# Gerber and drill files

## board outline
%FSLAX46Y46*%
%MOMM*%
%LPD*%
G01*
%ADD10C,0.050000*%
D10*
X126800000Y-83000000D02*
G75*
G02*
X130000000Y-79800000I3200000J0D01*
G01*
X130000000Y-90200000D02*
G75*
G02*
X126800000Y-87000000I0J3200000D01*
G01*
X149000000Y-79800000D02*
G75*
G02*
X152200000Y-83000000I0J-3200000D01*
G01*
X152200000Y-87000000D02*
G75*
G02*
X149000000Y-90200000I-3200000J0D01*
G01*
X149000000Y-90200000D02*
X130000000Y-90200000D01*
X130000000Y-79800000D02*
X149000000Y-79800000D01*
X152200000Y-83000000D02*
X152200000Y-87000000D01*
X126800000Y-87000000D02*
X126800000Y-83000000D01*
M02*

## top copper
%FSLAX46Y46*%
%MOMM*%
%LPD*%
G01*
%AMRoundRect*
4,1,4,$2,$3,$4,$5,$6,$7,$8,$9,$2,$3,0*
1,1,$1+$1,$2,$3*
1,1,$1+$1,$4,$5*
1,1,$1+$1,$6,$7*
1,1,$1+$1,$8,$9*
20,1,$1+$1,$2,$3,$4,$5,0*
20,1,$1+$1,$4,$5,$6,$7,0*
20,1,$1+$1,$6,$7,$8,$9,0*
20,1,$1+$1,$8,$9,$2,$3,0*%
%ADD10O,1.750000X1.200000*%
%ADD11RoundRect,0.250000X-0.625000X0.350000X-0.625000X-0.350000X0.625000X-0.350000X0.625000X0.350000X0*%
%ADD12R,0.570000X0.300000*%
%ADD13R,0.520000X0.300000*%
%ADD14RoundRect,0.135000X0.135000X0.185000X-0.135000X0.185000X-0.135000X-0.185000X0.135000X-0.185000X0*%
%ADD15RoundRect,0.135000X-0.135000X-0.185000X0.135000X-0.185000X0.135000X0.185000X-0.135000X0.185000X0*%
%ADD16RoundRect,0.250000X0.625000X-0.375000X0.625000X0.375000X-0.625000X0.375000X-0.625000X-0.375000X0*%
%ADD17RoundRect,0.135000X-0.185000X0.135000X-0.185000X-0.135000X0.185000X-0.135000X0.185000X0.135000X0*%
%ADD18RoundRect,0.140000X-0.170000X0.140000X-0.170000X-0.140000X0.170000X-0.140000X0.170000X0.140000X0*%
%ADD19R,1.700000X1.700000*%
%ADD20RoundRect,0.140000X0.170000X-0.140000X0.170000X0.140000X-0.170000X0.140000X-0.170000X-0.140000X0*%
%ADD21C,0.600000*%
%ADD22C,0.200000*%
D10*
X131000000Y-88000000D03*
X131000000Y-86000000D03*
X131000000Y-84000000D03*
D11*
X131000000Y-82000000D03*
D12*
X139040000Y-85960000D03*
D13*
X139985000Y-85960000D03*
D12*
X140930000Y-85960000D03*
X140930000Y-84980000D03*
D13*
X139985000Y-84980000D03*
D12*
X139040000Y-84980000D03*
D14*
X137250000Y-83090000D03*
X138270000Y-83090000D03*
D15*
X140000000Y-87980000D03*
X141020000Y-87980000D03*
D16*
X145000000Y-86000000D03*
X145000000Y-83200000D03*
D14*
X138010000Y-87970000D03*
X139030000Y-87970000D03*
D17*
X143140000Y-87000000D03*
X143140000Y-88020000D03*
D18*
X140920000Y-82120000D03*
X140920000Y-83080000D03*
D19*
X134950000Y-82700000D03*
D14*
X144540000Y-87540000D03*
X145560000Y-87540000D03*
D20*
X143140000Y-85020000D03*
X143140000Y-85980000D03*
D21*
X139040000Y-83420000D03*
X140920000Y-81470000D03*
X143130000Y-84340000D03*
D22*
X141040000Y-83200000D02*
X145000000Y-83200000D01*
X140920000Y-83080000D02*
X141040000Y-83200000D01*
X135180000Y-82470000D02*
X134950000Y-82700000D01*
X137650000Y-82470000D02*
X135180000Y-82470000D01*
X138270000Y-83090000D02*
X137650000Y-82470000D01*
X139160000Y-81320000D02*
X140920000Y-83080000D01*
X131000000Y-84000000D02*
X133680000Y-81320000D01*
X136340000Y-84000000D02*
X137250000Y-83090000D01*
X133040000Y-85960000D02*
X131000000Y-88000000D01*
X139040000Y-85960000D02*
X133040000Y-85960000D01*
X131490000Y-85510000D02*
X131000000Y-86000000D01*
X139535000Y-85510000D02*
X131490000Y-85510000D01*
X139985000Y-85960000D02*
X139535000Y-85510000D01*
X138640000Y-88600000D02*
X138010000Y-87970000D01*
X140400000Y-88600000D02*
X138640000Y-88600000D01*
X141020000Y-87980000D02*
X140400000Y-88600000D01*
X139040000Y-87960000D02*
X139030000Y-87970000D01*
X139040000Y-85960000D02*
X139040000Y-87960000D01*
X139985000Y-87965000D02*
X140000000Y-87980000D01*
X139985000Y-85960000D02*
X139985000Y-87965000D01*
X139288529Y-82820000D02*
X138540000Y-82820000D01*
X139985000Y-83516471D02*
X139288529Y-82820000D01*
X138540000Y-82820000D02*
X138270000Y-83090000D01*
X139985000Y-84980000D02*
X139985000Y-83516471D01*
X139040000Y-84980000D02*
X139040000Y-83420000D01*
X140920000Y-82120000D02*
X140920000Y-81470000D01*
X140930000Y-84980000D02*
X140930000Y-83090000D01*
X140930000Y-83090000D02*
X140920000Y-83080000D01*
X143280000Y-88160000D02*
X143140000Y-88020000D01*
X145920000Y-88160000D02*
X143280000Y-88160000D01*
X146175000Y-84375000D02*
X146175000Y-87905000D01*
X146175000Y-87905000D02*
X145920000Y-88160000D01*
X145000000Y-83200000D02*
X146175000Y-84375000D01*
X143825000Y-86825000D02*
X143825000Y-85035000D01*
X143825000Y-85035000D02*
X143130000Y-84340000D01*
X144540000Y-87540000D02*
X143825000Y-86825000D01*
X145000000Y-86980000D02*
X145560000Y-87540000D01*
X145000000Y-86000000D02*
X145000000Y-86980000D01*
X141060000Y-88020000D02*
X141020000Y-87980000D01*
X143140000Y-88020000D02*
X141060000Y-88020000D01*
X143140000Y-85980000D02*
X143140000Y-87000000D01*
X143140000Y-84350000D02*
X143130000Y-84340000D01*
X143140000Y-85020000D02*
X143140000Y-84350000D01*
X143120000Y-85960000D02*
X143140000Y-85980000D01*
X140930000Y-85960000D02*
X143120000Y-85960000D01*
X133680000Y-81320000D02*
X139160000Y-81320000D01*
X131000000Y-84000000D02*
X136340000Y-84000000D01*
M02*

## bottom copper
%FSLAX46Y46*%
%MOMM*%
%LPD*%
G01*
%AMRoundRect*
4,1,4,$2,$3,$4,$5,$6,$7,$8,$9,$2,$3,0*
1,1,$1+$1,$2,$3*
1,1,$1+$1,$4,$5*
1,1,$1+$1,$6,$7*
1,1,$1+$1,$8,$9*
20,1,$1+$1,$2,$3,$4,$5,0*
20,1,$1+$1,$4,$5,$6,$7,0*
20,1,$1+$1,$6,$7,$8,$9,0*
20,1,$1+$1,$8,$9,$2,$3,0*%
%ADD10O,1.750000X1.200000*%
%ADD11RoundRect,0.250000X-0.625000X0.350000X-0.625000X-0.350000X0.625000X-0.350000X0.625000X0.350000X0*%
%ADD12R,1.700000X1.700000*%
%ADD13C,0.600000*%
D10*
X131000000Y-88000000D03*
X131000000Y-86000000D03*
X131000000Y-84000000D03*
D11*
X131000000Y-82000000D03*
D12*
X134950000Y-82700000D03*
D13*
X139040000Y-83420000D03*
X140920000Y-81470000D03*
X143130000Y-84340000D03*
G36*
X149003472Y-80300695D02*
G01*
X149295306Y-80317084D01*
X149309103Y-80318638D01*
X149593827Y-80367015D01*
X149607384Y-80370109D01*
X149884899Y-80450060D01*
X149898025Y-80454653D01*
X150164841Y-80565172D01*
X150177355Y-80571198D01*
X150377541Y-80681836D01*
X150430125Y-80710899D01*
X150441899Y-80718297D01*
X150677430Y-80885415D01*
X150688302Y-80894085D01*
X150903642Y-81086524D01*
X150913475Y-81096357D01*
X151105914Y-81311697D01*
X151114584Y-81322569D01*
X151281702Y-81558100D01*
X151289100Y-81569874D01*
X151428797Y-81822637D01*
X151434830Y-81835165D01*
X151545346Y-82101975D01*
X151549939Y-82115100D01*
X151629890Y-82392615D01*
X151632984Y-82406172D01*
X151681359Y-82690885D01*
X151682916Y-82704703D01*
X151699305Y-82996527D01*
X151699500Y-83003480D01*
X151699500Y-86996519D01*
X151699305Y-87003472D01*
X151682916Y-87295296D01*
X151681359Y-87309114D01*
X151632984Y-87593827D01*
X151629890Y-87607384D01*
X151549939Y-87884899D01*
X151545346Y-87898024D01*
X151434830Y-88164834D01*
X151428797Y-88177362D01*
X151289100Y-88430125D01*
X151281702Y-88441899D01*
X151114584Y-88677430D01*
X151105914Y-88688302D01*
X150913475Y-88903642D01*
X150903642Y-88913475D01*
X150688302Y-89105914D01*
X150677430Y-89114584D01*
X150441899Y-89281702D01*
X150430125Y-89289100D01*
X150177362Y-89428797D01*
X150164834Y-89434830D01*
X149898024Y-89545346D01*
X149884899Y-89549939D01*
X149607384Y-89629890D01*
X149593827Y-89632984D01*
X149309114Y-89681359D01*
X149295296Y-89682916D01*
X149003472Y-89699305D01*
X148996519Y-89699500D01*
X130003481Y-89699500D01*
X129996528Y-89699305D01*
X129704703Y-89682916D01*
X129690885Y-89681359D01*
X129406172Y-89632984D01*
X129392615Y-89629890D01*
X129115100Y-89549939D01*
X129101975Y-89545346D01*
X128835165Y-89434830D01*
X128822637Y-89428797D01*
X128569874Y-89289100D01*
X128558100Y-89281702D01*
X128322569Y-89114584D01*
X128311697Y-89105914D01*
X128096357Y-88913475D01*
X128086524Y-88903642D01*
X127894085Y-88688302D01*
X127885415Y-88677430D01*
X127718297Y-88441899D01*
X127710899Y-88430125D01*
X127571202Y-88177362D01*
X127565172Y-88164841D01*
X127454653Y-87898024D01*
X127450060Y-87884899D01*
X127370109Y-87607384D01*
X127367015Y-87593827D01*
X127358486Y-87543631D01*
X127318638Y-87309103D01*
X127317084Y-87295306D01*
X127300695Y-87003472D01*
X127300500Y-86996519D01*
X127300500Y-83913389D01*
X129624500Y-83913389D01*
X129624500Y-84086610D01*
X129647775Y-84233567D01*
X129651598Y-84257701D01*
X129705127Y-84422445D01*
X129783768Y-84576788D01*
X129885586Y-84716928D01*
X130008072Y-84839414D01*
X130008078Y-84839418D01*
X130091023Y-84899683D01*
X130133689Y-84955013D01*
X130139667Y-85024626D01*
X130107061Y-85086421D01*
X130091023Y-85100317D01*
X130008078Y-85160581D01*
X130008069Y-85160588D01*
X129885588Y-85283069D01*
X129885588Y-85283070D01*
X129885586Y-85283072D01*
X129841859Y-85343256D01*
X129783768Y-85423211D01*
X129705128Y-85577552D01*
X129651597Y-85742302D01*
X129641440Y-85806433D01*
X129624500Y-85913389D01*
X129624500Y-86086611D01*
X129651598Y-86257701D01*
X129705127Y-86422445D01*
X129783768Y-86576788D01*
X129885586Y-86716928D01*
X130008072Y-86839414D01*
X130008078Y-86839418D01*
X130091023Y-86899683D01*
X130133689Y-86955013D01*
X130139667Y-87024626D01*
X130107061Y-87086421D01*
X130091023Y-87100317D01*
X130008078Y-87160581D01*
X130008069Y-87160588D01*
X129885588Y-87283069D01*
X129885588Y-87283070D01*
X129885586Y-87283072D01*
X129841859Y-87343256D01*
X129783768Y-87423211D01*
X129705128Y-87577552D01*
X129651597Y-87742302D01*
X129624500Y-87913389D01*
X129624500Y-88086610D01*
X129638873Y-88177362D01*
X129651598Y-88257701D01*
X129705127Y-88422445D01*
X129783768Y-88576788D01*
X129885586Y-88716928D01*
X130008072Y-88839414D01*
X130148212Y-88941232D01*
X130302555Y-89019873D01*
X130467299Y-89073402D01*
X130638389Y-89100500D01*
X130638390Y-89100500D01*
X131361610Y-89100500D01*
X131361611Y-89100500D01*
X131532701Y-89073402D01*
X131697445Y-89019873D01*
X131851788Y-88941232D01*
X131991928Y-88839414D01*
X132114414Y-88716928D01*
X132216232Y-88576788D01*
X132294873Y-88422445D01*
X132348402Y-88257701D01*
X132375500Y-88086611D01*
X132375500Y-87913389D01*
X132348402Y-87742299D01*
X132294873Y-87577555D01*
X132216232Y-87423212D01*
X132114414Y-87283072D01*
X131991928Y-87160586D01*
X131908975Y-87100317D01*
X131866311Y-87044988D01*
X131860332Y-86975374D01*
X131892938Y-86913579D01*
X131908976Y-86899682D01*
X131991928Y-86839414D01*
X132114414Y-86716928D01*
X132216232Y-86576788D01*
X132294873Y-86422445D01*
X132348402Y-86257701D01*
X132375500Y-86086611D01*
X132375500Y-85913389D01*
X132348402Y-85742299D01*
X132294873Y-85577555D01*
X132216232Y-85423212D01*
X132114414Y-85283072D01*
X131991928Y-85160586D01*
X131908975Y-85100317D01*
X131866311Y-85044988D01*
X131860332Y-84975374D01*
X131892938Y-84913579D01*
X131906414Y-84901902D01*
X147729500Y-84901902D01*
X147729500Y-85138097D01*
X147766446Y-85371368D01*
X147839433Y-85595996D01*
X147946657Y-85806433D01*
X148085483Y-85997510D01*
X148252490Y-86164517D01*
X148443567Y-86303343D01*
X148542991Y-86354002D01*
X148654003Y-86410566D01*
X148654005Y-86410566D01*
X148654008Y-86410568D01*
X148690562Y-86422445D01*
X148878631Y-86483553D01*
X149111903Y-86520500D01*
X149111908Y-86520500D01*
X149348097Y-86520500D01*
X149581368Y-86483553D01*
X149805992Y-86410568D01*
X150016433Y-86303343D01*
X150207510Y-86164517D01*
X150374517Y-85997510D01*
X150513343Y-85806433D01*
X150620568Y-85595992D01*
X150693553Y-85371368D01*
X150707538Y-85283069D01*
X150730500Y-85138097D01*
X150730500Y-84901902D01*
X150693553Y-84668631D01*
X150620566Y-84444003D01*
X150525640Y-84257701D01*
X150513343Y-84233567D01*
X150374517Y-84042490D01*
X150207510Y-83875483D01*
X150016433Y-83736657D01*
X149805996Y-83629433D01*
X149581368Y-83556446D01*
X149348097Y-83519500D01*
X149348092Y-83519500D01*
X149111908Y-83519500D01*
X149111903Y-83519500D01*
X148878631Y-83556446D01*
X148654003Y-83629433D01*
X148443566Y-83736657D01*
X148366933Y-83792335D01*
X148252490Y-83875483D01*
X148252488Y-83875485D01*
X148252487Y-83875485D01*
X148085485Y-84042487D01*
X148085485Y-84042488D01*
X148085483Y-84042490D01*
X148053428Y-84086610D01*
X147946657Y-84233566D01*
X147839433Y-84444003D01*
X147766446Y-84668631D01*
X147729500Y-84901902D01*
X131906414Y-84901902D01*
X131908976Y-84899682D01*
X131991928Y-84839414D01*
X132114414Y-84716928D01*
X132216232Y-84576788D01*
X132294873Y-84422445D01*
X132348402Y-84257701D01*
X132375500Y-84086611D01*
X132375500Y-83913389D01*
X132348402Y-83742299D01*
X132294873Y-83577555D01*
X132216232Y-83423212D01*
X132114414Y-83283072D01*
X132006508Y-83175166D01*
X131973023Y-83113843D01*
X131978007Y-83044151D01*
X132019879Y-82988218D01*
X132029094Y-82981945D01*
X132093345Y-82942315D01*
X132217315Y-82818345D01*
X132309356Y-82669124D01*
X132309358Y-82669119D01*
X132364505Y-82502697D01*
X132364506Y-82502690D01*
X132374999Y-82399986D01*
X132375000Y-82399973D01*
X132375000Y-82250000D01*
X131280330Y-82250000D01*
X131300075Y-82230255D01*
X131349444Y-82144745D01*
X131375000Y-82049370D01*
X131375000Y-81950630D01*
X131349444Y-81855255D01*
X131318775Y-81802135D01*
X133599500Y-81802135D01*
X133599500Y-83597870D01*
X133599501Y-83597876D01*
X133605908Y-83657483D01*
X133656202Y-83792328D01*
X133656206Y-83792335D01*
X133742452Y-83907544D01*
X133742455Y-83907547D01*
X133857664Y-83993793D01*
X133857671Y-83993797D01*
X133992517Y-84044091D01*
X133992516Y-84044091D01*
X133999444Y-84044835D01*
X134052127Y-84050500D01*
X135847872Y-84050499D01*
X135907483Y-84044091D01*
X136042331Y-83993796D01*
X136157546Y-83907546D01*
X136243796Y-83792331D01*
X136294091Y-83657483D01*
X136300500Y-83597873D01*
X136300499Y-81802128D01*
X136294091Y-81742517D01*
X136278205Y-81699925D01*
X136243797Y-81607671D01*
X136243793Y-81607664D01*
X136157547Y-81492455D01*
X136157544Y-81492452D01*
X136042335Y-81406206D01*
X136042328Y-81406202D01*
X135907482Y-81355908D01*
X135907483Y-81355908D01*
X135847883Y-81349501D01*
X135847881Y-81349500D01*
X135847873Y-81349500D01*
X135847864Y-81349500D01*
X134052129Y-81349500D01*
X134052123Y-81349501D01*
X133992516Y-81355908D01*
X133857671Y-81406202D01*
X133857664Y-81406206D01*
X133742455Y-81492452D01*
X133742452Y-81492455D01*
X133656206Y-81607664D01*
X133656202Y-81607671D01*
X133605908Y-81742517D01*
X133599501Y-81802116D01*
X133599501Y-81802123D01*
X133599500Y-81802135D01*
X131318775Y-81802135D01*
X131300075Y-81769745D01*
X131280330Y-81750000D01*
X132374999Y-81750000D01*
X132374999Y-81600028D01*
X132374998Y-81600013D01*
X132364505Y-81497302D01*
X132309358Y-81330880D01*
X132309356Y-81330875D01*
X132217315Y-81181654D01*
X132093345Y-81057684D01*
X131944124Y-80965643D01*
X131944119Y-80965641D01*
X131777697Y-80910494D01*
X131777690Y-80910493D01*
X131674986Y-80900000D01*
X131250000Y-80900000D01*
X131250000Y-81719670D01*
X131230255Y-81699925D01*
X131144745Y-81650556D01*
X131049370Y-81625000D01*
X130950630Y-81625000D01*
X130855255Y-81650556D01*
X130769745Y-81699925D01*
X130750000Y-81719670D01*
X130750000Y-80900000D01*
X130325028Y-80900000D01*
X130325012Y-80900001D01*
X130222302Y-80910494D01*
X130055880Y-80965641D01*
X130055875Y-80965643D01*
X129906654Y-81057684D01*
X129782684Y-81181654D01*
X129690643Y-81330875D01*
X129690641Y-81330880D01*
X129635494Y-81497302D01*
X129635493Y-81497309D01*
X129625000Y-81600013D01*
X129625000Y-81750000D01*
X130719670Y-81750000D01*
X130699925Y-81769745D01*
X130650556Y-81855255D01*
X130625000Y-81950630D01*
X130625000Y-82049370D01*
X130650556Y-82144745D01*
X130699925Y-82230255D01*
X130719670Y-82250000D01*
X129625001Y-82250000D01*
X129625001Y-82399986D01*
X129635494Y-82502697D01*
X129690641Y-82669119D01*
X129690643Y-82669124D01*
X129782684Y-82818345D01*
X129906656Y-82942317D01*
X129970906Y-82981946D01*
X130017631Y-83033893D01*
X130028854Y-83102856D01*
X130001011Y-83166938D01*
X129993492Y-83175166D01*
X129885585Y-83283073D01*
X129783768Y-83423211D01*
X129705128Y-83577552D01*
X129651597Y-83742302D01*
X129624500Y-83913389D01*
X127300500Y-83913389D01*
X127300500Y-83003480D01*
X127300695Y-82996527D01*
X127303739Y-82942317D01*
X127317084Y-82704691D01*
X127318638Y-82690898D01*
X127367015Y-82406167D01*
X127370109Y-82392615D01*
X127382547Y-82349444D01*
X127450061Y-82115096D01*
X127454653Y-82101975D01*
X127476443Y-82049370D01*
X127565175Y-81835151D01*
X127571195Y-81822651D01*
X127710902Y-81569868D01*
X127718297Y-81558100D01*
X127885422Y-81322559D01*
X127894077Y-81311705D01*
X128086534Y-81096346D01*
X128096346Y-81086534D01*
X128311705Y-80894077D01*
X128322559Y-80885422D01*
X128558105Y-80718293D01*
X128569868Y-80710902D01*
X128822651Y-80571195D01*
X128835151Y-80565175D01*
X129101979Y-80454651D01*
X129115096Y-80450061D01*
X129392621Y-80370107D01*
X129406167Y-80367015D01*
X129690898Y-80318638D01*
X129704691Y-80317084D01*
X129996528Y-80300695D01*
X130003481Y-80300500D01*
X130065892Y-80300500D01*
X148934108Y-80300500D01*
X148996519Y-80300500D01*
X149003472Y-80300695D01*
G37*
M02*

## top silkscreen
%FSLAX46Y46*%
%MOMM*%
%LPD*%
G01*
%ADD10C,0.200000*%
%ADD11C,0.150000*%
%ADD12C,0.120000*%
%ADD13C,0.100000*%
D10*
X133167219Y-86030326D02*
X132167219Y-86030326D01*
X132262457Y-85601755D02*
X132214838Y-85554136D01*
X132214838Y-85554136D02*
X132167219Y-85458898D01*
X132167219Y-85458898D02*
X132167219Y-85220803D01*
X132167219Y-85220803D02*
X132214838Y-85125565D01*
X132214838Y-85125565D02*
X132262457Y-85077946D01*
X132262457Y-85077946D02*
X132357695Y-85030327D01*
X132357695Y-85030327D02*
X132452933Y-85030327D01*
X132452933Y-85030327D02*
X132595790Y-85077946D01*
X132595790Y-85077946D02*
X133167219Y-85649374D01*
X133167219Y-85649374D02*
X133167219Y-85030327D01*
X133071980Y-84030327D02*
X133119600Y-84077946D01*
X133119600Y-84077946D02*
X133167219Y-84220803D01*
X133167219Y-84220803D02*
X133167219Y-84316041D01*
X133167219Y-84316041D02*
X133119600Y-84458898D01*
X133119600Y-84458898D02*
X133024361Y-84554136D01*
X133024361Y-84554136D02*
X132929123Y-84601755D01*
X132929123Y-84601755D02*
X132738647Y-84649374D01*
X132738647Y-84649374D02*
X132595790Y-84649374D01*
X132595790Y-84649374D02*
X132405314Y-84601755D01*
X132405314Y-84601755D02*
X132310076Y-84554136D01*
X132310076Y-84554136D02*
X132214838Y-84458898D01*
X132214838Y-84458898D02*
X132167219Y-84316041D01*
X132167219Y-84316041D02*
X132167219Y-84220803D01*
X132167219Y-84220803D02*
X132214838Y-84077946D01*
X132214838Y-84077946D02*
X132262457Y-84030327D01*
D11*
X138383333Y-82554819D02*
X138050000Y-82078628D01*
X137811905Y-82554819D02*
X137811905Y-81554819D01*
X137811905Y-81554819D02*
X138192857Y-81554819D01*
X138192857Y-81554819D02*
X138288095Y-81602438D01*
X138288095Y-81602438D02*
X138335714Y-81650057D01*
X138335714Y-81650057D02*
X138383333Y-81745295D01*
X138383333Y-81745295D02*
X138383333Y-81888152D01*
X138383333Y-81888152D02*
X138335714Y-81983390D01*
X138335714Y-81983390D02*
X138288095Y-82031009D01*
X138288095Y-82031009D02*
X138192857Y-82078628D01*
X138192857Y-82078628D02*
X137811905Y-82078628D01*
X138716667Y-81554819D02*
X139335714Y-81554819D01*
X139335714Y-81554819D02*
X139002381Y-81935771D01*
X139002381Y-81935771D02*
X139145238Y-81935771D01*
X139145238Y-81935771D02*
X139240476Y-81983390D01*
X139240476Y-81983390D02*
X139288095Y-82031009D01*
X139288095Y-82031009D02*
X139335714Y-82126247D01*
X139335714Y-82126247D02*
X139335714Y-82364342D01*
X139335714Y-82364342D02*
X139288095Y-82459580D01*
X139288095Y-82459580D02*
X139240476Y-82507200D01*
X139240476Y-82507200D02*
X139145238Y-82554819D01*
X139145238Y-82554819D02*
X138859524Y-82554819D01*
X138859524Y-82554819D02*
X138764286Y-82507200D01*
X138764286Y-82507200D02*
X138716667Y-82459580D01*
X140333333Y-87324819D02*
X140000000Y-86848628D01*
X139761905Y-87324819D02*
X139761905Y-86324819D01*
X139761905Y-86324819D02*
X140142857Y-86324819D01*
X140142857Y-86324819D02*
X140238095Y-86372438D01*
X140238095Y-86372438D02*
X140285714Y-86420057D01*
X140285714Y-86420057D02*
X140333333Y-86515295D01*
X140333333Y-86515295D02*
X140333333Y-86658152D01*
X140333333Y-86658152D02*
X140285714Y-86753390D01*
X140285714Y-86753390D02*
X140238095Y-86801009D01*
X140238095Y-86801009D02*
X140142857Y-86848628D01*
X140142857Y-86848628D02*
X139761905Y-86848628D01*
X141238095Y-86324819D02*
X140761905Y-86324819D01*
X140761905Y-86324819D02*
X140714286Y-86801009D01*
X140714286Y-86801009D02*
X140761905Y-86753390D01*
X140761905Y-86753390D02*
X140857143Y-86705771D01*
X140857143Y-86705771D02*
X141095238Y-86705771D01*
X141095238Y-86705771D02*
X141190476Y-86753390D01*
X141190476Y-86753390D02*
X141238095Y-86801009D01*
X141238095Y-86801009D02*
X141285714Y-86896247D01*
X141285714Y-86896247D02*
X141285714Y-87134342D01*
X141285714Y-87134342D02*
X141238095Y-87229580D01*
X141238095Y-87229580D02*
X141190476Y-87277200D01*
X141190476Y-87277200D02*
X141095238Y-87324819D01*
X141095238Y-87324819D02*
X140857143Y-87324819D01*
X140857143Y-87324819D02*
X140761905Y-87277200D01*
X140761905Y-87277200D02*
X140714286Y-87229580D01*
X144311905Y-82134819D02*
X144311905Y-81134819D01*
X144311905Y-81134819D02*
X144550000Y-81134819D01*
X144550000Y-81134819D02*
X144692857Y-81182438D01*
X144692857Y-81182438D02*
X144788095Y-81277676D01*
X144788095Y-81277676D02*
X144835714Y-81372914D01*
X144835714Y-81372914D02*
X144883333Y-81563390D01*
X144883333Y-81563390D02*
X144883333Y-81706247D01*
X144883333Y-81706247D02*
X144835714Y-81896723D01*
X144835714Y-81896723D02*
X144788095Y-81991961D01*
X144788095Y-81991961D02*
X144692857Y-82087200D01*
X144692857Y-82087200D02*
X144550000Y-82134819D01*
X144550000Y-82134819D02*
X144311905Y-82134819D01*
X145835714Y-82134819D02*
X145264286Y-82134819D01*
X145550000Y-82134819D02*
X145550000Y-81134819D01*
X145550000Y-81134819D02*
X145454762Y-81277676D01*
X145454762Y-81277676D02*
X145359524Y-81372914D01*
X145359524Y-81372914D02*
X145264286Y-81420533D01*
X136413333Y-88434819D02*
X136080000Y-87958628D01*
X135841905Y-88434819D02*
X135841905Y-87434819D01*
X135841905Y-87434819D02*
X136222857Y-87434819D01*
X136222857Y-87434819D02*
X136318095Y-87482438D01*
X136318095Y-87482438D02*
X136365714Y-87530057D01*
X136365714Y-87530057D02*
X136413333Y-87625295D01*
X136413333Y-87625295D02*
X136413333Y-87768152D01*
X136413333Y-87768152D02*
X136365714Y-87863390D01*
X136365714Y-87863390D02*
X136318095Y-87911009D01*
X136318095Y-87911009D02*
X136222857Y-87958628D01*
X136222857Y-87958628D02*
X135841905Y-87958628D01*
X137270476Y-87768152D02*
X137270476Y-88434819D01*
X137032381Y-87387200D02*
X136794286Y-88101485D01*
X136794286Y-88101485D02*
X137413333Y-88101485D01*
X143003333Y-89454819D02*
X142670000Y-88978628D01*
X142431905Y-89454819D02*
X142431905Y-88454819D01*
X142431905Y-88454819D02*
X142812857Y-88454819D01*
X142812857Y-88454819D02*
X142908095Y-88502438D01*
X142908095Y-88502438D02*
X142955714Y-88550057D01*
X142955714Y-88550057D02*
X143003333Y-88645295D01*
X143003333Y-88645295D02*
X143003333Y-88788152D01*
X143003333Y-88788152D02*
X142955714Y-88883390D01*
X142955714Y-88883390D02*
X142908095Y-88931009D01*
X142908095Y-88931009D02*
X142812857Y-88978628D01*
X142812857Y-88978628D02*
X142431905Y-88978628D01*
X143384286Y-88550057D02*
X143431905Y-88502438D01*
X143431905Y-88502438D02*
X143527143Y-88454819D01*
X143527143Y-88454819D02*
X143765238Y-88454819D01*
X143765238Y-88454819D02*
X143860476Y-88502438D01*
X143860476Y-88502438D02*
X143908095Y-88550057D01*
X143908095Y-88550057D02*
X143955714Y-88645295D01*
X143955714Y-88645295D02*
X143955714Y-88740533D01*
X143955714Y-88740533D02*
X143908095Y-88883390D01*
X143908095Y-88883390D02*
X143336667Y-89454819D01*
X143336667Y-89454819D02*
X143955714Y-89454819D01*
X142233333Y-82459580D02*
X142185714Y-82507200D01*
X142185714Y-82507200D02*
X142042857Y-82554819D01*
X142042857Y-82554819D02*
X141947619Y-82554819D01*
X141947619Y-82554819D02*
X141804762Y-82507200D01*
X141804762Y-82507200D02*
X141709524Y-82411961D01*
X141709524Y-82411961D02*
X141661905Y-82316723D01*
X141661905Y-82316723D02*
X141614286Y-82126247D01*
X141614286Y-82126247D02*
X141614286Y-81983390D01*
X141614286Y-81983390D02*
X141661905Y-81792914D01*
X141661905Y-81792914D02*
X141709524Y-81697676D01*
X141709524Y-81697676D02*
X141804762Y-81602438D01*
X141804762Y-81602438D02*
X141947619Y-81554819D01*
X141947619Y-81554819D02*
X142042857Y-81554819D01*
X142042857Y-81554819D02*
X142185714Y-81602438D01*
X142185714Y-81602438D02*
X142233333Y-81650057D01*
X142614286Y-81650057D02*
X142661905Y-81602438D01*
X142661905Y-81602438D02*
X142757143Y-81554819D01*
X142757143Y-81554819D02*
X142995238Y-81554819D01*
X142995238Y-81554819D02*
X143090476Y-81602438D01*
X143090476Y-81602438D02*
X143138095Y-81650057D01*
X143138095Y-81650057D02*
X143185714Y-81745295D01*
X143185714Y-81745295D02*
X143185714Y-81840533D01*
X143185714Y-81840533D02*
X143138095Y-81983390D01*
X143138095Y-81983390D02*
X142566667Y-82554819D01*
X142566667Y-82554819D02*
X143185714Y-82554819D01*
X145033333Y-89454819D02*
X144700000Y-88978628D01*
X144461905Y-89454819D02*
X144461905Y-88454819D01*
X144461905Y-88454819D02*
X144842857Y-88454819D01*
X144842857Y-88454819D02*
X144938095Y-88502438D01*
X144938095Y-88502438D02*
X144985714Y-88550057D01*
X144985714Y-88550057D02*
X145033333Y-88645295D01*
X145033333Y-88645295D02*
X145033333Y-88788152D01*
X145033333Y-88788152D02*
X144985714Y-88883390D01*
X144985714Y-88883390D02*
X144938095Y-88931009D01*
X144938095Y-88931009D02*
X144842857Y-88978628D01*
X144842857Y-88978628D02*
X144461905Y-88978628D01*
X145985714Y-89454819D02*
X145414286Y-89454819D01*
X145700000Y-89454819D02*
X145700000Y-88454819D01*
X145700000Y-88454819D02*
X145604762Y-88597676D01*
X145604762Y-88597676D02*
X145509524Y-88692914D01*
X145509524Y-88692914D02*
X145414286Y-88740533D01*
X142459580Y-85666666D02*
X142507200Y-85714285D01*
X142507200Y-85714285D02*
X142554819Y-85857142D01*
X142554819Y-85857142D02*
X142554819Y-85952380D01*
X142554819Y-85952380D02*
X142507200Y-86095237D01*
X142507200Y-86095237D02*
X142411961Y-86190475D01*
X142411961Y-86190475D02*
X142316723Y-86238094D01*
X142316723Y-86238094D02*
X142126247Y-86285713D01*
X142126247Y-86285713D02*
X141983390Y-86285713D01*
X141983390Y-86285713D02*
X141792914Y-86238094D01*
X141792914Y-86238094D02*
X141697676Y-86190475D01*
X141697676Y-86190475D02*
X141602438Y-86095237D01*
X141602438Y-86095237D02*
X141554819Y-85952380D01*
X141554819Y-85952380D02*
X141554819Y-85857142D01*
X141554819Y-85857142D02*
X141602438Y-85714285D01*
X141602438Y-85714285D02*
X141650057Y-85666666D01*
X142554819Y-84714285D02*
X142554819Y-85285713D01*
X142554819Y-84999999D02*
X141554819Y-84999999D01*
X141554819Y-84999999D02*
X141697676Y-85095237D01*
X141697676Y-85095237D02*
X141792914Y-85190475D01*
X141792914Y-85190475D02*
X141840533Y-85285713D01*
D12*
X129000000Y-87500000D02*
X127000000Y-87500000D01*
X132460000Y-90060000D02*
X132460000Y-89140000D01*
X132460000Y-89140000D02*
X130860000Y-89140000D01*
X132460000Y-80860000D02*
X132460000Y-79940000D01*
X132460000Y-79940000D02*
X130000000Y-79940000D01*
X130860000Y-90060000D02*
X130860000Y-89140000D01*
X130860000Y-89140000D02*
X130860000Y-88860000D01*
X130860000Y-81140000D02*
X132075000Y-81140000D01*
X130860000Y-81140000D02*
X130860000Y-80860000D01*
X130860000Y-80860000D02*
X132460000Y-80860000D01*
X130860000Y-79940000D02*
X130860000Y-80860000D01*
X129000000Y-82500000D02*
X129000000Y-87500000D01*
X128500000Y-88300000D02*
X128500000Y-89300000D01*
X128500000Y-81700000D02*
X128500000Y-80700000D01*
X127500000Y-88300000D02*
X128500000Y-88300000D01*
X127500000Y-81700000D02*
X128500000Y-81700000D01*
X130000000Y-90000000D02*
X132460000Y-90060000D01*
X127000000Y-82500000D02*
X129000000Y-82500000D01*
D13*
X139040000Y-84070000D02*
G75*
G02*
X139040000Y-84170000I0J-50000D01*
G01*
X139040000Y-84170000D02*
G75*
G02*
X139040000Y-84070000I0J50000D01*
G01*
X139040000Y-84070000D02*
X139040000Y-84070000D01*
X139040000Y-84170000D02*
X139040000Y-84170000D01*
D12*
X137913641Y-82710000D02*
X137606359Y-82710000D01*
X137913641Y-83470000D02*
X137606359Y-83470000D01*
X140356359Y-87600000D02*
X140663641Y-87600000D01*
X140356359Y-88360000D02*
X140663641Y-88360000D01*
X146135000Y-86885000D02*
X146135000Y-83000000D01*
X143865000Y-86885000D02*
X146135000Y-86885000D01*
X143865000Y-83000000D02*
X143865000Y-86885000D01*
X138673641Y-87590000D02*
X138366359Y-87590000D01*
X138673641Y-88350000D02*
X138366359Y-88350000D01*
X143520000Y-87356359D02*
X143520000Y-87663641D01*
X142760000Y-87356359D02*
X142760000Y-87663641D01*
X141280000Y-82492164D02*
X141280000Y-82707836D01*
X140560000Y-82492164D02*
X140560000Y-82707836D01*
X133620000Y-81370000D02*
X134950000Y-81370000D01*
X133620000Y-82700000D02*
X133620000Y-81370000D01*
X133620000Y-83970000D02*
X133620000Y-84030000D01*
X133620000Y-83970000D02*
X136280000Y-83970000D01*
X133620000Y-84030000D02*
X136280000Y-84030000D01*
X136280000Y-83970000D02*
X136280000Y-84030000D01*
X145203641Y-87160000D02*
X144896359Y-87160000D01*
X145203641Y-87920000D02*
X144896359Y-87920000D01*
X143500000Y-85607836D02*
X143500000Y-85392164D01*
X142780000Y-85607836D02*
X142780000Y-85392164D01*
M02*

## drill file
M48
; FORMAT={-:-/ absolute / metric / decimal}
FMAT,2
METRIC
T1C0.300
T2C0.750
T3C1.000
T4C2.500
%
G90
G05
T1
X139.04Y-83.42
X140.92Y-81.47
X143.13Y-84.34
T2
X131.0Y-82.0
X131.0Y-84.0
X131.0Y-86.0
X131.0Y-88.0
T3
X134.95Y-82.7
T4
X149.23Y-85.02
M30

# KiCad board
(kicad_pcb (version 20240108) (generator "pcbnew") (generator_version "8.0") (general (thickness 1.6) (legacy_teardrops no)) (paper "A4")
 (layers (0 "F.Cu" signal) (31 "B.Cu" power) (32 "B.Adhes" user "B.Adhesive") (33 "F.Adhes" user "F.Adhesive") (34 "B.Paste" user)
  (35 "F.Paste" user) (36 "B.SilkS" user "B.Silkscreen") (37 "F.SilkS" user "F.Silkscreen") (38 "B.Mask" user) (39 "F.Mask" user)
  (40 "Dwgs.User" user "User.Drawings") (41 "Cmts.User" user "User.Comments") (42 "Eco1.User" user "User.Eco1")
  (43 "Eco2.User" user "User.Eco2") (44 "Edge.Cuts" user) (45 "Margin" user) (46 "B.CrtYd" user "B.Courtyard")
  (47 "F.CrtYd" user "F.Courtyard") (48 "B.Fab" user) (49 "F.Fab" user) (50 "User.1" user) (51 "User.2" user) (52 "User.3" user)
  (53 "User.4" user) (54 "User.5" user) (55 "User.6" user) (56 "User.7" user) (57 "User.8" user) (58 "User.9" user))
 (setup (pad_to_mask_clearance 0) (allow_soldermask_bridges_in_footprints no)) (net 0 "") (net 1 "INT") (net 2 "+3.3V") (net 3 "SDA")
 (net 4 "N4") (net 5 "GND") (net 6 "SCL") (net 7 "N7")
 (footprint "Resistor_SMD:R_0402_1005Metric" (layer "F.Cu") (at 137.76 83.09 180)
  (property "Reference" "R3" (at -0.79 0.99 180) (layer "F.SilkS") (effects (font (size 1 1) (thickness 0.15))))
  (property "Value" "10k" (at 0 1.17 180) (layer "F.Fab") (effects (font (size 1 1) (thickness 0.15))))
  (fp_line (start -0.153641 0.38) (end 0.153641 0.38) (stroke (width 0.12) (type solid)) (layer "F.SilkS"))
  (fp_line (start -0.153641 -0.38) (end 0.153641 -0.38) (stroke (width 0.12) (type solid)) (layer "F.SilkS"))
  (pad "1" smd roundrect (at -0.51 0 180) (size 0.54 0.64) (layers "F.Cu" "F.Paste" "F.Mask") (roundrect_rratio 0.25) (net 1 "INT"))
  (pad "2" smd roundrect (at 0.51 0 180) (size 0.54 0.64) (layers "F.Cu" "F.Paste" "F.Mask") (roundrect_rratio 0.25) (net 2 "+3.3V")))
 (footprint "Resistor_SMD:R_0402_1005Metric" (layer "F.Cu") (at 140.51 87.98)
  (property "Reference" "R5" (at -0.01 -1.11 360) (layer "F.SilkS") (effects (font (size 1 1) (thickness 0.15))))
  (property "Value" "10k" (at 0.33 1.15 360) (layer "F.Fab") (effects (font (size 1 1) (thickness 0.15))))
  (fp_line (start -0.153641 -0.38) (end 0.153641 -0.38) (stroke (width 0.12) (type solid)) (layer "F.SilkS"))
  (fp_line (start -0.153641 0.38) (end 0.153641 0.38) (stroke (width 0.12) (type solid)) (layer "F.SilkS"))
  (pad "1" smd roundrect (at -0.51 0) (size 0.54 0.64) (layers "F.Cu" "F.Paste" "F.Mask") (roundrect_rratio 0.25) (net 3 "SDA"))
  (pad "2" smd roundrect (at 0.51 0) (size 0.54 0.64) (layers "F.Cu" "F.Paste" "F.Mask") (roundrect_rratio 0.25) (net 2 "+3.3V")))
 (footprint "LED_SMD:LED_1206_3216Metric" (layer "F.Cu") (at 145 84.6 90)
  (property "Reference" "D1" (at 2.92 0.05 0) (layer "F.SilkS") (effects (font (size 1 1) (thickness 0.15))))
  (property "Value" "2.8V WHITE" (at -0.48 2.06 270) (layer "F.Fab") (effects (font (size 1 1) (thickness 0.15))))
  (fp_line (start 1.6 -1.135) (end -2.285 -1.135) (stroke (width 0.12) (type solid)) (layer "F.SilkS"))
  (fp_line (start -2.285 -1.135) (end -2.285 1.135) (stroke (width 0.12) (type solid)) (layer "F.SilkS"))
  (fp_line (start -2.285 1.135) (end 1.6 1.135) (stroke (width 0.12) (type solid)) (layer "F.SilkS"))
  (pad "1" smd roundrect (at -1.4 0 90) (size 1.25 1.75) (layers "F.Cu" "F.Paste" "F.Mask") (roundrect_rratio 0.2) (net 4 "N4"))
  (pad "2" smd roundrect (at 1.4 0 90) (size 1.25 1.75) (layers "F.Cu" "F.Paste" "F.Mask") (roundrect_rratio 0.2) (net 2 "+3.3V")))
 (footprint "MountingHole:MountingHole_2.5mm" (layer "F.Cu") (at 149.23 85.02)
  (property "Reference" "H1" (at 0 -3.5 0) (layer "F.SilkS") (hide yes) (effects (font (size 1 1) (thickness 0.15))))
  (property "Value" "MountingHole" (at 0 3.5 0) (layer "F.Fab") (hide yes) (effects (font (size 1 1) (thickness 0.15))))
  (pad "" np_thru_hole circle (at 0 0) (size 2.5 2.5) (drill 2.5) (layers "*.Cu" "*.Mask")))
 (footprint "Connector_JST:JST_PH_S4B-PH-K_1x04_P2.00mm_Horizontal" (layer "F.Cu") (at 131 82 -90)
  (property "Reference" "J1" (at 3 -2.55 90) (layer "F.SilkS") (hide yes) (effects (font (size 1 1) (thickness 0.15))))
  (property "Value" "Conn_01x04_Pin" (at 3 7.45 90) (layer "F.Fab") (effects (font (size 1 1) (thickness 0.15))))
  (fp_line (start 0.5 4) (end 0.5 2) (stroke (width 0.12) (type solid)) (layer "F.SilkS"))
  (fp_line (start -0.3 3.5) (end -0.3 2.5) (stroke (width 0.12) (type solid)) (layer "F.SilkS"))
  (fp_line (start 6.3 3.5) (end 6.3 2.5) (stroke (width 0.12) (type solid)) (layer "F.SilkS"))
  (fp_line (start -0.3 2.5) (end -1.3 2.5) (stroke (width 0.12) (type solid)) (layer "F.SilkS"))
  (fp_line (start 6.3 2.5) (end 7.3 2.5) (stroke (width 0.12) (type solid)) (layer "F.SilkS"))
  (fp_line (start 0.5 2) (end 5.5 2) (stroke (width 0.12) (type solid)) (layer "F.SilkS"))
  (fp_line (start 5.5 2) (end 5.5 4) (stroke (width 0.12) (type solid)) (layer "F.SilkS"))
  (fp_line (start 8 1) (end 8.06 -1.46) (stroke (width 0.12) (type solid)) (layer "F.SilkS"))
  (fp_line (start -2.06 0.14) (end -1.14 0.14) (stroke (width 0.12) (type solid)) (layer "F.SilkS"))
  (fp_line (start -1.14 0.14) (end -1.14 -1.46) (stroke (width 0.12) (type solid)) (layer "F.SilkS"))
  (fp_line (start -0.86 0.14) (end -1.14 0.14) (stroke (width 0.12) (type solid)) (layer "F.SilkS"))
  (fp_line (start -0.86 0.14) (end -0.86 -1.075) (stroke (width 0.12) (type solid)) (layer "F.SilkS"))
  (fp_line (start 7.14 0.14) (end 6.86 0.14) (stroke (width 0.12) (type solid)) (layer "F.SilkS"))
  (fp_line (start 8.06 0.14) (end 7.14 0.14) (stroke (width 0.12) (type solid)) (layer "F.SilkS"))
  (fp_line (start -2.06 -1.46) (end -2.06 1) (stroke (width 0.12) (type solid)) (layer "F.SilkS"))
  (fp_line (start -1.14 -1.46) (end -2.06 -1.46) (stroke (width 0.12) (type solid)) (layer "F.SilkS"))
  (fp_line (start 7.14 -1.46) (end 7.14 0.14) (stroke (width 0.12) (type solid)) (layer "F.SilkS"))
  (fp_line (start 8.06 -1.46) (end 7.14 -1.46) (stroke (width 0.12) (type solid)) (layer "F.SilkS"))
  (pad "1" thru_hole roundrect (at 0 0 270) (size 1.2 1.75) (drill 0.75) (layers "*.Cu" "*.Mask") (remove_unused_layers no)
   (roundrect_rratio 0.208333) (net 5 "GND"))
  (pad "2" thru_hole oval (at 2 0 270) (size 1.2 1.75) (drill 0.75) (layers "*.Cu" "*.Mask") (remove_unused_layers no) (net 2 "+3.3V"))
  (pad "3" thru_hole oval (at 4 0 270) (size 1.2 1.75) (drill 0.75) (layers "*.Cu" "*.Mask") (remove_unused_layers no) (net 3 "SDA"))
  (pad "4" thru_hole oval (at 6 0 270) (size 1.2 1.75) (drill 0.75) (layers "*.Cu" "*.Mask") (remove_unused_layers no) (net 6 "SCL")))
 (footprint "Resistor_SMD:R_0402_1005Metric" (layer "F.Cu") (at 138.52 87.97 180)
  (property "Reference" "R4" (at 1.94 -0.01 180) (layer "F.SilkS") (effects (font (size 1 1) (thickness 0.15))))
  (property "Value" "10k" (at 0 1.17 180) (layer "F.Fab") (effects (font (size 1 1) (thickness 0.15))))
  (fp_line (start -0.153641 0.38) (end 0.153641 0.38) (stroke (width 0.12) (type solid)) (layer "F.SilkS"))
  (fp_line (start -0.153641 -0.38) (end 0.153641 -0.38) (stroke (width 0.12) (type solid)) (layer "F.SilkS"))
  (pad "1" smd roundrect (at -0.51 0 180) (size 0.54 0.64) (layers "F.Cu" "F.Paste" "F.Mask") (roundrect_rratio 0.25) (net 6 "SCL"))
  (pad "2" smd roundrect (at 0.51 0 180) (size 0.54 0.64) (layers "F.Cu" "F.Paste" "F.Mask") (roundrect_rratio 0.25) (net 2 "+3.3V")))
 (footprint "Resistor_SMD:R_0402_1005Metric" (layer "F.Cu") (at 143.14 87.51 -90)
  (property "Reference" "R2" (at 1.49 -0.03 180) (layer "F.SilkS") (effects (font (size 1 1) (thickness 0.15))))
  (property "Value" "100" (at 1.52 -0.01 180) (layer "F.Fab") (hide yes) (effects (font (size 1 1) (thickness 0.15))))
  (fp_line (start -0.153641 0.38) (end 0.153641 0.38) (stroke (width 0.12) (type solid)) (layer "F.SilkS"))
  (fp_line (start -0.153641 -0.38) (end 0.153641 -0.38) (stroke (width 0.12) (type solid)) (layer "F.SilkS"))
  (pad "1" smd roundrect (at -0.51 0 270) (size 0.54 0.64) (layers "F.Cu" "F.Paste" "F.Mask") (roundrect_rratio 0.25) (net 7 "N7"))
  (pad "2" smd roundrect (at 0.51 0 270) (size 0.54 0.64) (layers "F.Cu" "F.Paste" "F.Mask") (roundrect_rratio 0.25) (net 2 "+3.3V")))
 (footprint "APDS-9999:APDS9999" (layer "F.Cu") (at 139.985 85.47 90)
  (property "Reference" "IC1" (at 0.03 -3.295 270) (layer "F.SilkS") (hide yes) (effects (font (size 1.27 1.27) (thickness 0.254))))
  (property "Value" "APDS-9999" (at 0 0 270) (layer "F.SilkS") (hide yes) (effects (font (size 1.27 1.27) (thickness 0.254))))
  (fp_line (start 1.4 -0.945) (end 1.4 -0.945) (stroke (width 0.1) (type solid)) (layer "F.SilkS"))
  (fp_line (start 1.3 -0.945) (end 1.3 -0.945) (stroke (width 0.1) (type solid)) (layer "F.SilkS"))
  (fp_arc (start 1.4 -0.945) (mid 1.35 -0.895) (end 1.3 -0.945) (stroke (width 0.1) (type solid)) (layer "F.SilkS"))
  (fp_arc (start 1.3 -0.945) (mid 1.35 -0.995) (end 1.4 -0.945) (stroke (width 0.1) (type solid)) (layer "F.SilkS"))
  (pad "1" smd rect (at 0.49 -0.945 90) (size 0.3 0.57) (layers "F.Cu" "F.Paste" "F.Mask") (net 5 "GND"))
  (pad "2" smd rect (at 0.49 0 90) (size 0.3 0.52) (layers "F.Cu" "F.Paste" "F.Mask") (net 1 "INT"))
  (pad "3" smd rect (at 0.49 0.945 90) (size 0.3 0.57) (layers "F.Cu" "F.Paste" "F.Mask") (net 2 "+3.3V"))
  (pad "4" smd rect (at -0.49 0.945 90) (size 0.3 0.57) (layers "F.Cu" "F.Paste" "F.Mask") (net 7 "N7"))
  (pad "5" smd rect (at -0.49 0 90) (size 0.3 0.52) (layers "F.Cu" "F.Paste" "F.Mask") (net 3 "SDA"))
  (pad "6" smd rect (at -0.49 -0.945 90) (size 0.3 0.57) (layers "F.Cu" "F.Paste" "F.Mask") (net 6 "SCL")))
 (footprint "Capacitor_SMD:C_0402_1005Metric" (layer "F.Cu") (at 140.92 82.6 -90)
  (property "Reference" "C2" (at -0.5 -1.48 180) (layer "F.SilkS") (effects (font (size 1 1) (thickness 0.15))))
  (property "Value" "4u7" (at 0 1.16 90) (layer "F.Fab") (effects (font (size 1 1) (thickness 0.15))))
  (fp_line (start -0.107836 0.36) (end 0.107836 0.36) (stroke (width 0.12) (type solid)) (layer "F.SilkS"))
  (fp_line (start -0.107836 -0.36) (end 0.107836 -0.36) (stroke (width 0.12) (type solid)) (layer "F.SilkS"))
  (pad "1" smd roundrect (at -0.48 0 270) (size 0.56 0.62) (layers "F.Cu" "F.Paste" "F.Mask") (roundrect_rratio 0.25) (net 5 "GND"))
  (pad "2" smd roundrect (at 0.48 0 270) (size 0.56 0.62) (layers "F.Cu" "F.Paste" "F.Mask") (roundrect_rratio 0.25) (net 2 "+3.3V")))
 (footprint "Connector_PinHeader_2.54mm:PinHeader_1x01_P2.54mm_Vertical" (layer "F.Cu") (at 134.95 82.7)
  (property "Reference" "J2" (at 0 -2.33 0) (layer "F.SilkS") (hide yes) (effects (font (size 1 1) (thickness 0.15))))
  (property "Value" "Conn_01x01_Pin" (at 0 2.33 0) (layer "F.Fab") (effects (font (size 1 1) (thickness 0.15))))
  (fp_line (start -1.33 -1.33) (end 0 -1.33) (stroke (width 0.12) (type solid)) (layer "F.SilkS"))
  (fp_line (start -1.33 0) (end -1.33 -1.33) (stroke (width 0.12) (type solid)) (layer "F.SilkS"))
  (fp_line (start -1.33 1.27) (end -1.33 1.33) (stroke (width 0.12) (type solid)) (layer "F.SilkS"))
  (fp_line (start -1.33 1.27) (end 1.33 1.27) (stroke (width 0.12) (type solid)) (layer "F.SilkS"))
  (fp_line (start -1.33 1.33) (end 1.33 1.33) (stroke (width 0.12) (type solid)) (layer "F.SilkS"))
  (fp_line (start 1.33 1.27) (end 1.33 1.33) (stroke (width 0.12) (type solid)) (layer "F.SilkS"))
  (pad "1" thru_hole rect (at 0 0) (size 1.7 1.7) (drill 1) (layers "*.Cu" "*.Mask") (remove_unused_layers no) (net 1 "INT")))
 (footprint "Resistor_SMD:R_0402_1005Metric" (layer "F.Cu") (at 145.05 87.54 180)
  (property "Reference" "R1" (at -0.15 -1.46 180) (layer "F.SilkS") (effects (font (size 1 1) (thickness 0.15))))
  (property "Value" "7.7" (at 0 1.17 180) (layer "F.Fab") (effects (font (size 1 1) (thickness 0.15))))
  (fp_line (start -0.153641 0.38) (end 0.153641 0.38) (stroke (width 0.12) (type solid)) (layer "F.SilkS"))
  (fp_line (start -0.153641 -0.38) (end 0.153641 -0.38) (stroke (width 0.12) (type solid)) (layer "F.SilkS"))
  (pad "1" smd roundrect (at -0.51 0 180) (size 0.54 0.64) (layers "F.Cu" "F.Paste" "F.Mask") (roundrect_rratio 0.25) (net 4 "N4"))
  (pad "2" smd roundrect (at 0.51 0 180) (size 0.54 0.64) (layers "F.Cu" "F.Paste" "F.Mask") (roundrect_rratio 0.25) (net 5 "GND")))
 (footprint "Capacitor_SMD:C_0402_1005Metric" (layer "F.Cu") (at 143.14 85.5 90)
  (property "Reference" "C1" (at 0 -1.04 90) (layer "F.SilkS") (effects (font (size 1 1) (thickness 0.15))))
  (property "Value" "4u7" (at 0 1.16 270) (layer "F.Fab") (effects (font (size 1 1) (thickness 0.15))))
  (fp_line (start -0.107836 -0.36) (end 0.107836 -0.36) (stroke (width 0.12) (type solid)) (layer "F.SilkS"))
  (fp_line (start -0.107836 0.36) (end 0.107836 0.36) (stroke (width 0.12) (type solid)) (layer "F.SilkS"))
  (pad "1" smd roundrect (at -0.48 0 90) (size 0.56 0.62) (layers "F.Cu" "F.Paste" "F.Mask") (roundrect_rratio 0.25) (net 7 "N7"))
  (pad "2" smd roundrect (at 0.48 0 90) (size 0.56 0.62) (layers "F.Cu" "F.Paste" "F.Mask") (roundrect_rratio 0.25) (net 5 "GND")))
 (gr_arc (start 149 79.8) (mid 151.262742 80.737258) (end 152.2 83) (stroke (width 0.05) (type default)) (layer "Edge.Cuts"))
 (gr_line (start 149 90.2) (end 130 90.2) (stroke (width 0.05) (type default)) (layer "Edge.Cuts"))
 (gr_arc (start 130 90.2) (mid 127.737258 89.262742) (end 126.8 87) (stroke (width 0.05) (type default)) (layer "Edge.Cuts"))
 (gr_line (start 130 79.8) (end 149 79.8) (stroke (width 0.05) (type default)) (layer "Edge.Cuts"))
 (gr_arc (start 152.2 87) (mid 151.262742 89.262742) (end 149 90.2) (stroke (width 0.05) (type default)) (layer "Edge.Cuts"))
 (gr_arc (start 126.8 83) (mid 127.737258 80.737258) (end 130 79.8) (stroke (width 0.05) (type default)) (layer "Edge.Cuts"))
 (gr_line (start 152.2 83) (end 152.2 87) (stroke (width 0.05) (type default)) (layer "Edge.Cuts"))
 (gr_line (start 126.8 87) (end 126.8 83) (stroke (width 0.05) (type default)) (layer "Edge.Cuts"))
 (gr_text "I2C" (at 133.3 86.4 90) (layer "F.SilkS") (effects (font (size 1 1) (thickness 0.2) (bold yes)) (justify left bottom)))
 (segment (start 143.14 85.02) (end 143.14 84.35) (width 0.2) (layer "F.Cu") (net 5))
 (segment (start 140.92 82.12) (end 140.92 81.47) (width 0.2) (layer "F.Cu") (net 5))
 (segment (start 143.825 85.035) (end 143.13 84.34) (width 0.2) (layer "F.Cu") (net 5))
 (segment (start 139.04 84.98) (end 139.04 83.42) (width 0.2) (layer "F.Cu") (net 5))
 (segment (start 143.825 86.825) (end 143.825 85.035) (width 0.2) (layer "F.Cu") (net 5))
 (segment (start 144.54 87.54) (end 143.825 86.825) (width 0.2) (layer "F.Cu") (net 5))
 (segment (start 143.14 84.35) (end 143.13 84.34) (width 0.2) (layer "F.Cu") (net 5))
 (via (at 143.13 84.34) (size 0.6) (drill 0.3) (layers "F.Cu" "B.Cu") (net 5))
 (via (at 140.92 81.47) (size 0.6) (drill 0.3) (layers "F.Cu" "B.Cu") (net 5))
 (via (at 139.04 83.42) (size 0.6) (drill 0.3) (layers "F.Cu" "B.Cu") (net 5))
 (segment (start 143.12 85.96) (end 143.14 85.98) (width 0.2) (layer "F.Cu") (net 7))
 (segment (start 140.93 85.96) (end 143.12 85.96) (width 0.2) (layer "F.Cu") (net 7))
 (segment (start 143.14 85.98) (end 143.14 87) (width 0.2) (layer "F.Cu") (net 7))
 (segment (start 141.04 83.2) (end 145 83.2) (width 0.2) (layer "F.Cu") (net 2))
 (segment (start 140.92 83.08) (end 141.04 83.2) (width 0.2) (layer "F.Cu") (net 2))
 (segment (start 145.92 88.16) (end 143.28 88.16) (width 0.2) (layer "F.Cu") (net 2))
 (segment (start 146.175 87.905) (end 145.92 88.16) (width 0.2) (layer "F.Cu") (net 2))
 (segment (start 138.64 88.6) (end 138.01 87.97) (width 0.2) (layer "F.Cu") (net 2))
 (segment (start 140.4 88.6) (end 138.64 88.6) (width 0.2) (layer "F.Cu") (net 2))
 (segment (start 146.175 84.375) (end 146.175 87.905) (width 0.2) (layer "F.Cu") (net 2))
 (segment (start 139.16 81.32) (end 140.92 83.08) (width 0.2) (layer "F.Cu") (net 2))
 (segment (start 143.28 88.16) (end 143.14 88.02) (width 0.2) (layer "F.Cu") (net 2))
 (segment (start 140.93 83.09) (end 140.92 83.08) (width 0.2) (layer "F.Cu") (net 2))
 (segment (start 141.02 87.98) (end 140.4 88.6) (width 0.2) (layer "F.Cu") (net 2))
 (segment (start 131 84) (end 136.34 84) (width 0.2) (layer "F.Cu") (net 2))
 (segment (start 131 84) (end 133.68 81.32) (width 0.2) (layer "F.Cu") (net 2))
 (segment (start 136.34 84) (end 137.25 83.09) (width 0.2) (layer "F.Cu") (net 2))
 (segment (start 133.68 81.32) (end 139.16 81.32) (width 0.2) (layer "F.Cu") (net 2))
 (segment (start 145 83.2) (end 146.175 84.375) (width 0.2) (layer "F.Cu") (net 2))
 (segment (start 141.06 88.02) (end 141.02 87.98) (width 0.2) (layer "F.Cu") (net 2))
 (segment (start 140.93 84.98) (end 140.93 83.09) (width 0.2) (layer "F.Cu") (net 2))
 (segment (start 143.14 88.02) (end 141.06 88.02) (width 0.2) (layer "F.Cu") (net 2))
 (segment (start 145 86.98) (end 145.56 87.54) (width 0.2) (layer "F.Cu") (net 4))
 (segment (start 145 86) (end 145 86.98) (width 0.2) (layer "F.Cu") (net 4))
 (segment (start 139.04 85.96) (end 139.04 87.96) (width 0.2) (layer "F.Cu") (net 6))
 (segment (start 139.04 87.96) (end 139.03 87.97) (width 0.2) (layer "F.Cu") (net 6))
 (segment (start 133.04 85.96) (end 131 88) (width 0.2) (layer "F.Cu") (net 6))
 (segment (start 139.04 85.96) (end 133.04 85.96) (width 0.2) (layer "F.Cu") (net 6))
 (segment (start 139.985 87.965) (end 140 87.98) (width 0.2) (layer "F.Cu") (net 3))
 (segment (start 131.49 85.51) (end 131 86) (width 0.2) (layer "F.Cu") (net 3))
 (segment (start 139.535 85.51) (end 131.49 85.51) (width 0.2) (layer "F.Cu") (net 3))
 (segment (start 139.985 85.96) (end 139.985 87.965) (width 0.2) (layer "F.Cu") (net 3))
 (segment (start 139.985 85.96) (end 139.535 85.51) (width 0.2) (layer "F.Cu") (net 3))
 (segment (start 139.985 83.516471) (end 139.288529 82.82) (width 0.2) (layer "F.Cu") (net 1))
 (segment (start 139.288529 82.82) (end 138.54 82.82) (width 0.2) (layer "F.Cu") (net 1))
 (segment (start 138.27 83.09) (end 137.65 82.47) (width 0.2) (layer "F.Cu") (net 1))
 (segment (start 137.65 82.47) (end 135.18 82.47) (width 0.2) (layer "F.Cu") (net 1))
 (segment (start 135.18 82.47) (end 134.95 82.7) (width 0.2) (layer "F.Cu") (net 1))
 (segment (start 139.985 84.98) (end 139.985 83.516471) (width 0.2) (layer "F.Cu") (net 1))
 (segment (start 138.54 82.82) (end 138.27 83.09) (width 0.2) (layer "F.Cu") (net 1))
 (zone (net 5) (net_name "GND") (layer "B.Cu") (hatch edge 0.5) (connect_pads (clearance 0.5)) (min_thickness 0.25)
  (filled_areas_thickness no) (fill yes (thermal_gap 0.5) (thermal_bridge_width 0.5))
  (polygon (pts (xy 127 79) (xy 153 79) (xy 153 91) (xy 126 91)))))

